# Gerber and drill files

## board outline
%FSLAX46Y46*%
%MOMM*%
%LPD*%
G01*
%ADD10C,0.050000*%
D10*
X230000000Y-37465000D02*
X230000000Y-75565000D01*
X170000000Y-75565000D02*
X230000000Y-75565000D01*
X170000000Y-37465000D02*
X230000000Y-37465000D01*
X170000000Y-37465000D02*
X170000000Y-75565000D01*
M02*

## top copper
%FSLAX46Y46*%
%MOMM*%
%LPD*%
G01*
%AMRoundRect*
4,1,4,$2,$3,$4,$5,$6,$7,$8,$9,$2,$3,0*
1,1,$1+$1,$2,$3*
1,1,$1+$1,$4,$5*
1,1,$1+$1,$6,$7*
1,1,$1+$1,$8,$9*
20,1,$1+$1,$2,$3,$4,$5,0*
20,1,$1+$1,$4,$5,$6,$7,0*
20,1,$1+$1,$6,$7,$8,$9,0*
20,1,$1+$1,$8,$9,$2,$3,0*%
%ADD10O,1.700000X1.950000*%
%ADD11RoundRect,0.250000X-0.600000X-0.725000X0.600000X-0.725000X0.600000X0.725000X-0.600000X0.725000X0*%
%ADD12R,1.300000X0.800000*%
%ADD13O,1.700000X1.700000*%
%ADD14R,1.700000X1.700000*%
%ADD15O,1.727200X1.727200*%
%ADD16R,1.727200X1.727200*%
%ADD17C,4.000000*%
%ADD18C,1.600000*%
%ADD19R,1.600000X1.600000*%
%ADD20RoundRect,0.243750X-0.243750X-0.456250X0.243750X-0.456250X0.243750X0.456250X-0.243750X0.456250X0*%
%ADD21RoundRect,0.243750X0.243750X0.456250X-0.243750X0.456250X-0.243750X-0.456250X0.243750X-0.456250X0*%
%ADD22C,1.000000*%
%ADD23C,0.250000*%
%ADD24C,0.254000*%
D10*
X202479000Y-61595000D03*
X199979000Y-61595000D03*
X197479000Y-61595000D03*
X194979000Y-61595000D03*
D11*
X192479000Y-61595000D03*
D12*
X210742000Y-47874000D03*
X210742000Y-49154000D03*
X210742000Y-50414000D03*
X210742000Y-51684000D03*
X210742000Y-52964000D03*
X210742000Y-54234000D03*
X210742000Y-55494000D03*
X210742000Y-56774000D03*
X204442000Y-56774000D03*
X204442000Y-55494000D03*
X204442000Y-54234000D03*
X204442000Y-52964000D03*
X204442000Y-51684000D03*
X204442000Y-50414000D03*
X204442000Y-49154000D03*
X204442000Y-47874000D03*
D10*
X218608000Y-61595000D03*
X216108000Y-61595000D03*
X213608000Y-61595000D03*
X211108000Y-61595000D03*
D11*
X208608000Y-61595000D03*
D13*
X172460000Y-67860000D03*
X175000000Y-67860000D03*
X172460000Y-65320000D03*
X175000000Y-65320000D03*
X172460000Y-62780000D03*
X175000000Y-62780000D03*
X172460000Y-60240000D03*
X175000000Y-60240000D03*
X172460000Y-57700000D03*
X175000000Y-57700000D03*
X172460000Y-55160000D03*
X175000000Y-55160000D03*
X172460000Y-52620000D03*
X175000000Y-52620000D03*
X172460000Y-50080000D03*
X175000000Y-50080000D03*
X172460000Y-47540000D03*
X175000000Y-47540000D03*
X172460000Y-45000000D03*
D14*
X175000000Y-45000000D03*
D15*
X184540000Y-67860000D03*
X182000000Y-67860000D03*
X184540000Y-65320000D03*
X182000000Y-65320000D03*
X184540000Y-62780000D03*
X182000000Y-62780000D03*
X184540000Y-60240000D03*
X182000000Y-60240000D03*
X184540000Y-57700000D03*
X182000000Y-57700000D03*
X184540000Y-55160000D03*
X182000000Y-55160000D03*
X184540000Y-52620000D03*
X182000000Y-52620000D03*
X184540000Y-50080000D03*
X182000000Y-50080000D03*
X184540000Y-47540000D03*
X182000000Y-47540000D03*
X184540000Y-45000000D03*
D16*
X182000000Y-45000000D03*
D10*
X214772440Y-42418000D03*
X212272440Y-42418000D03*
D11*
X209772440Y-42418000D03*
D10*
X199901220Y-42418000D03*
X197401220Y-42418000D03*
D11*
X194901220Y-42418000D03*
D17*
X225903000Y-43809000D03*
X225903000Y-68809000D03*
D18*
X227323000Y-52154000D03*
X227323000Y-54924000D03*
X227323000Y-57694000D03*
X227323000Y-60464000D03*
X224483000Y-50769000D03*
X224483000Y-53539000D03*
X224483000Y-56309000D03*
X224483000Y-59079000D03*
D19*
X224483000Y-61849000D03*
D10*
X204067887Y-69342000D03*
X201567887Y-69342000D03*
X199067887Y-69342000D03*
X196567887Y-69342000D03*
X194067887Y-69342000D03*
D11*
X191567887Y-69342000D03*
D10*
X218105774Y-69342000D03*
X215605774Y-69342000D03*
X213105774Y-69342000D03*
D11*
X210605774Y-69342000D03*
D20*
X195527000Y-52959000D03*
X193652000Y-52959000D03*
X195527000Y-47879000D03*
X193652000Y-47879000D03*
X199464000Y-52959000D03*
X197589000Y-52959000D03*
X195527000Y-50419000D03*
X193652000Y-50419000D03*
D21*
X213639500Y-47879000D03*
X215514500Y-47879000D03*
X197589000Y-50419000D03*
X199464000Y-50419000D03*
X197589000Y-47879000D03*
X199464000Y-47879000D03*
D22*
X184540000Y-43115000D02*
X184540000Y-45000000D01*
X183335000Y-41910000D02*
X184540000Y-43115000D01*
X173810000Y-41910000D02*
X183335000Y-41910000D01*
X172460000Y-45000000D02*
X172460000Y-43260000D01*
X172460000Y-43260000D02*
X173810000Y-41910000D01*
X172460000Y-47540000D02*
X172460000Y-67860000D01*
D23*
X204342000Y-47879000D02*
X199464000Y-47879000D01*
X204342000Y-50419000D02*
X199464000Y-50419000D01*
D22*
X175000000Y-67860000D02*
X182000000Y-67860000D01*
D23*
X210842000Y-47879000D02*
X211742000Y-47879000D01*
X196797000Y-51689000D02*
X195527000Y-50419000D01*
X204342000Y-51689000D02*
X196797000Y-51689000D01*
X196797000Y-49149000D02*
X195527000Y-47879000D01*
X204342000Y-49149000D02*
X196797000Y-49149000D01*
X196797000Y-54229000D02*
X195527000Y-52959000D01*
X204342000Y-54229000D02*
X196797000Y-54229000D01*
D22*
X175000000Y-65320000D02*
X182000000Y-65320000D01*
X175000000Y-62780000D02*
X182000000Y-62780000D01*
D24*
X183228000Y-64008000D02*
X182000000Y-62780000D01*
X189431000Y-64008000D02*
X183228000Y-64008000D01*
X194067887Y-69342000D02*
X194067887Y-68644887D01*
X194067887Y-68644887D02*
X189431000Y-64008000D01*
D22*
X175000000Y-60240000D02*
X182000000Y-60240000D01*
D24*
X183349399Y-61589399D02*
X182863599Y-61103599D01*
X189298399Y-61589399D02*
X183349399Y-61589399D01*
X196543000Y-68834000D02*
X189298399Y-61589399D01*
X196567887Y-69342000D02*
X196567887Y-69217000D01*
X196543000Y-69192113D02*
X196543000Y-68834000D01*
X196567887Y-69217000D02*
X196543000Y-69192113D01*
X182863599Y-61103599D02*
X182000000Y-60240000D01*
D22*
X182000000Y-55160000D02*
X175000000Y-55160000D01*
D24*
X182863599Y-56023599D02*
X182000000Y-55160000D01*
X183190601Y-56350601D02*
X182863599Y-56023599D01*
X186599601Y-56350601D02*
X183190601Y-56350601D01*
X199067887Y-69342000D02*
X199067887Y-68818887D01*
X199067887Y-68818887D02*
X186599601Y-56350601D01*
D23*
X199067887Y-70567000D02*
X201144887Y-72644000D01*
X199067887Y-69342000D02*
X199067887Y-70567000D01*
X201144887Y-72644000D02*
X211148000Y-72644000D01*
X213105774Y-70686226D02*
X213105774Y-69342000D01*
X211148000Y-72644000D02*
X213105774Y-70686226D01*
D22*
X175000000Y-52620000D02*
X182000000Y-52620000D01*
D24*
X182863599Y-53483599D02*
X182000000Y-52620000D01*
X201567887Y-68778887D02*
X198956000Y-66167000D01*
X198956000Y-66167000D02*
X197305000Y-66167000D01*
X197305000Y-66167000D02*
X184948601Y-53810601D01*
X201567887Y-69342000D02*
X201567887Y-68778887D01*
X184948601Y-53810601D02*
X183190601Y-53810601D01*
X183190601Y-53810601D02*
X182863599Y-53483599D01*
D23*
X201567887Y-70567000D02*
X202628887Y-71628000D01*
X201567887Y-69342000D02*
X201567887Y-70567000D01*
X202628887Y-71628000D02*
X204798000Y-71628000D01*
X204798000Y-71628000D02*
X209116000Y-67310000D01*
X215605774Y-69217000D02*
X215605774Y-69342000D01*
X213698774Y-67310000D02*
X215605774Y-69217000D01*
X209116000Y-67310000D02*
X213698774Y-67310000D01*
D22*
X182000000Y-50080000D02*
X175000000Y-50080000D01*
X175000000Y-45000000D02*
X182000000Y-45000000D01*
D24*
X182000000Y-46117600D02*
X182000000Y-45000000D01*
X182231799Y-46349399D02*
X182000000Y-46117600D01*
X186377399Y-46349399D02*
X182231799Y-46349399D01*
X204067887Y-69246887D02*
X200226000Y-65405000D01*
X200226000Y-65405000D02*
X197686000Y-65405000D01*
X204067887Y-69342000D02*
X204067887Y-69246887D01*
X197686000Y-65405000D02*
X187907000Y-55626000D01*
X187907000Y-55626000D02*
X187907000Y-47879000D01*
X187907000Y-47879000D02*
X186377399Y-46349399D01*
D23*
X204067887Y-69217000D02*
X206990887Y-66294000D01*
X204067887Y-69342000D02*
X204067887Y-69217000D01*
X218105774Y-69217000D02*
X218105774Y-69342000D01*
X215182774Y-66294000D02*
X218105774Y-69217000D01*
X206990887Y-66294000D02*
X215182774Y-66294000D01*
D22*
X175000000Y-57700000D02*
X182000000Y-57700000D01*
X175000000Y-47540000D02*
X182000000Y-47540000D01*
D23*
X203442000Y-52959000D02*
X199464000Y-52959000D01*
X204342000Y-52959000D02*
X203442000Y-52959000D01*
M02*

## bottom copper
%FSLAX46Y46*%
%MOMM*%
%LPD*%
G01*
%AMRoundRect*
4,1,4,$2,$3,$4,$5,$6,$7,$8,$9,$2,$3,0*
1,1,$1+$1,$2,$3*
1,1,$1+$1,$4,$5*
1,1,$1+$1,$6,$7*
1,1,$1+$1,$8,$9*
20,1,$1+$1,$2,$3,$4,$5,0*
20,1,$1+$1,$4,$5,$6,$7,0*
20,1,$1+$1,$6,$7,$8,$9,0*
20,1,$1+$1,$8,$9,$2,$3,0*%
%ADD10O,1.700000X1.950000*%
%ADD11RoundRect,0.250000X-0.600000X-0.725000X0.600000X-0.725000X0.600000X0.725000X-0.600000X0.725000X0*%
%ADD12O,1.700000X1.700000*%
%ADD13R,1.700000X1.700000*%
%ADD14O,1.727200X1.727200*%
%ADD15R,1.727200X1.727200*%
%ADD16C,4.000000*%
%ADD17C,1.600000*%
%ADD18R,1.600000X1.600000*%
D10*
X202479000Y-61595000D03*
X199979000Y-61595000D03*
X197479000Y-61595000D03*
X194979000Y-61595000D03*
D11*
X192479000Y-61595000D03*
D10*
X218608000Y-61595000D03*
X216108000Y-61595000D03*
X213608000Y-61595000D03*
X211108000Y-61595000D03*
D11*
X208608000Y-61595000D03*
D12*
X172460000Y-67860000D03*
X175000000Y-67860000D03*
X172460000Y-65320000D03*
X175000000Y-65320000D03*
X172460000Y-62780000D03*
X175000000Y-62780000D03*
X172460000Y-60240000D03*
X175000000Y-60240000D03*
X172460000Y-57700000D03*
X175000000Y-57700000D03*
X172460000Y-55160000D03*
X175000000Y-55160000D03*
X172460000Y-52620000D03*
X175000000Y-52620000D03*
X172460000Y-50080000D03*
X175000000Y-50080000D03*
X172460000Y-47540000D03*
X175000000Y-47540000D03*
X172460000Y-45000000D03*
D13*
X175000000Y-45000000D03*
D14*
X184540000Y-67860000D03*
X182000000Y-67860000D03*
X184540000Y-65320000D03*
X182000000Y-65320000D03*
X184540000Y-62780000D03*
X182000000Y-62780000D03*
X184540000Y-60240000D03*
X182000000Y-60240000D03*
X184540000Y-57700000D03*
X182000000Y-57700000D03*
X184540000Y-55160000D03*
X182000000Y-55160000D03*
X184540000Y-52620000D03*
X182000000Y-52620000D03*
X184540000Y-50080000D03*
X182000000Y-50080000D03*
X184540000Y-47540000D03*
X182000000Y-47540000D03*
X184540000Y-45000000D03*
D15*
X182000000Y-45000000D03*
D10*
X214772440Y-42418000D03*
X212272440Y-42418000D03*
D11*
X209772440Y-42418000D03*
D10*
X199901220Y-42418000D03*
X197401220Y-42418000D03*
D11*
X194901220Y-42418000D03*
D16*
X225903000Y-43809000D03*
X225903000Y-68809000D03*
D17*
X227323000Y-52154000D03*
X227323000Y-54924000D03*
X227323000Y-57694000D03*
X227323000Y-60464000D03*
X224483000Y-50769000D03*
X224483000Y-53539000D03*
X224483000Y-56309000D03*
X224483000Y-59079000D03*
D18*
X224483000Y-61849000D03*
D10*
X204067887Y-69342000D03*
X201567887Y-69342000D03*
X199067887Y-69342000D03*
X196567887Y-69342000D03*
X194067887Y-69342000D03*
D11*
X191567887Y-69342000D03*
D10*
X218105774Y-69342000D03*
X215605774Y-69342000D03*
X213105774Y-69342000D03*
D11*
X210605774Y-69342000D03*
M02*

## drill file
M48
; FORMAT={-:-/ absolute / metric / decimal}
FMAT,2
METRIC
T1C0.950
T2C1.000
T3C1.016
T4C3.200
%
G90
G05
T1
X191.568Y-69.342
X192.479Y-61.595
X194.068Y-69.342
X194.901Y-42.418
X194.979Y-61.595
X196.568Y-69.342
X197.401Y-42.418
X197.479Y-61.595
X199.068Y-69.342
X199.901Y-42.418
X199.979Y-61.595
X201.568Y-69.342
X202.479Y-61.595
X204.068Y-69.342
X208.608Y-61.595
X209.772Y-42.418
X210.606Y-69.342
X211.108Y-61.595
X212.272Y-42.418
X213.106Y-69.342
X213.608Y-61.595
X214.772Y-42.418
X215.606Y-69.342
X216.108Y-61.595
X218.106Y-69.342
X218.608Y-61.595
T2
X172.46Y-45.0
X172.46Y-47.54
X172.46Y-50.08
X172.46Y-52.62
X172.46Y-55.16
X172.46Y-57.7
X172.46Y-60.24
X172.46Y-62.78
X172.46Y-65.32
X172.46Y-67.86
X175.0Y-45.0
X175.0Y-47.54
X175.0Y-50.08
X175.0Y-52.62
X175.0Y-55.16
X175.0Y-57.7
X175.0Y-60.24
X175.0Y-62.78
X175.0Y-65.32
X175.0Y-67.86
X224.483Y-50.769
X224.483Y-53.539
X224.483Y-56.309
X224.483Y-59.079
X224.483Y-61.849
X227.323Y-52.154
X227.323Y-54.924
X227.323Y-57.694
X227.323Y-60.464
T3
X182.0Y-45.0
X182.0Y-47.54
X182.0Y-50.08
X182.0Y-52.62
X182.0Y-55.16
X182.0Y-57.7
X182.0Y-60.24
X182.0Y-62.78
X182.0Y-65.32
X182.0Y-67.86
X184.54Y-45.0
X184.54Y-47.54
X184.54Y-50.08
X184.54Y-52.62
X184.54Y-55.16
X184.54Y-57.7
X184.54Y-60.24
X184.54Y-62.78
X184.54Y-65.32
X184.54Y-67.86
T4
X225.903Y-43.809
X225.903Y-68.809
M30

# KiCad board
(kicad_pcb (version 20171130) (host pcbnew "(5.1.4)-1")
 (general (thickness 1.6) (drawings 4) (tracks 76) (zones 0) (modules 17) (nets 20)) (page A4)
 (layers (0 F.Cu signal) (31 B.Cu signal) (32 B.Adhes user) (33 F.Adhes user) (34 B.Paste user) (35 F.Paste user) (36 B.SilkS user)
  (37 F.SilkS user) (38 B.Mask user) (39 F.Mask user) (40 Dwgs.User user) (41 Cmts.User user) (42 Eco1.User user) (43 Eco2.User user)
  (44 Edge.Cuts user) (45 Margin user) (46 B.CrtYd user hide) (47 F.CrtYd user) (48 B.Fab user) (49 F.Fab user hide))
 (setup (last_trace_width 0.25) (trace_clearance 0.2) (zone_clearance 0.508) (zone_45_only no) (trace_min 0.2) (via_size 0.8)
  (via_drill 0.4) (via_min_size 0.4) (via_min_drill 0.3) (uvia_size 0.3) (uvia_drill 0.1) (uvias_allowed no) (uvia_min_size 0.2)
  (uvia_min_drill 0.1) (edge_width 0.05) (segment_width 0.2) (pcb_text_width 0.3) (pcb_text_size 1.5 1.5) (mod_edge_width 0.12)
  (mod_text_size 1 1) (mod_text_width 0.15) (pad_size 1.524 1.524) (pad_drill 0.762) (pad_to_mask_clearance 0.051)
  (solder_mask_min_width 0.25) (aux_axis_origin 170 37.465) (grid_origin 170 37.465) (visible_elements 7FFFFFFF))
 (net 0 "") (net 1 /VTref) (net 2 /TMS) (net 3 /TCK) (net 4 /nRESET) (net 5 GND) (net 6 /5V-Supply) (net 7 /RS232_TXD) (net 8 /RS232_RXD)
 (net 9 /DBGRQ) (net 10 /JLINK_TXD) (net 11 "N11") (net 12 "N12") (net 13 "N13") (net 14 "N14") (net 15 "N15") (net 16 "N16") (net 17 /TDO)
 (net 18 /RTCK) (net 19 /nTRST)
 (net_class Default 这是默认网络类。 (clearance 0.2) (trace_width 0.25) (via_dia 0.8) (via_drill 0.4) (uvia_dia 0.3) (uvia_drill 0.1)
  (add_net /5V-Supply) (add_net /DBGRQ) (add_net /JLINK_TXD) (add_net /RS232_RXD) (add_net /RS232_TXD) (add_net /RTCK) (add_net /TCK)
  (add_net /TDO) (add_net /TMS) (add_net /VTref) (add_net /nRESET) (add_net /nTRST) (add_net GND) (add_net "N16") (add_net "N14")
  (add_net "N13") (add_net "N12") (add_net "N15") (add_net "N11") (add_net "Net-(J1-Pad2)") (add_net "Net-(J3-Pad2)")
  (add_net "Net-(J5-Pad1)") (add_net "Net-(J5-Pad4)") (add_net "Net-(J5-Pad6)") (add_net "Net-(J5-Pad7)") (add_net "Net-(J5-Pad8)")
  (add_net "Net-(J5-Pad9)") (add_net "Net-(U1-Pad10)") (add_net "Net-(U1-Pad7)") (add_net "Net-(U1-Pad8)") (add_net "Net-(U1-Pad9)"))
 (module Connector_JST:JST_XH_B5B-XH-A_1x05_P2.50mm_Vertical (layer F.Cu) (at 192.479 61.595)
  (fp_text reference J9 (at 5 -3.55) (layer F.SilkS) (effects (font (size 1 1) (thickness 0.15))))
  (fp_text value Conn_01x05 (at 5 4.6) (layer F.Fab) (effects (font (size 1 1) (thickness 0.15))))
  (pad 5 thru_hole oval (at 10 0) (size 1.7 1.95) (drill 0.95) (layers *.Cu *.Mask) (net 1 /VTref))
  (pad 4 thru_hole oval (at 7.5 0) (size 1.7 1.95) (drill 0.95) (layers *.Cu *.Mask) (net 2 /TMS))
  (pad 3 thru_hole oval (at 5 0) (size 1.7 1.95) (drill 0.95) (layers *.Cu *.Mask) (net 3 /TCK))
  (pad 2 thru_hole oval (at 2.5 0) (size 1.7 1.95) (drill 0.95) (layers *.Cu *.Mask) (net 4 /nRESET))
  (pad 1 thru_hole roundrect (at 0 0) (size 1.7 1.95) (drill 0.95) (layers *.Cu *.Mask) (roundrect_rratio 0.147059) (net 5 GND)))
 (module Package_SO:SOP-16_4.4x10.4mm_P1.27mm (layer F.Cu) (at 207.592 52.324)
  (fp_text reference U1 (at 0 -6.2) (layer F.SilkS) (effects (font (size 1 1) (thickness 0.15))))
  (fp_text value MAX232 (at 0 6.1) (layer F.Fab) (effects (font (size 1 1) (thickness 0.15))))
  (pad 16 smd rect (at 3.15 -4.45) (size 1.3 0.8) (layers F.Cu F.Paste F.Mask) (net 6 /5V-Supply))
  (pad 15 smd rect (at 3.15 -3.17) (size 1.3 0.8) (layers F.Cu F.Paste F.Mask) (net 5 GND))
  (pad 14 smd rect (at 3.15 -1.91) (size 1.3 0.8) (layers F.Cu F.Paste F.Mask) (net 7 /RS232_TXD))
  (pad 13 smd rect (at 3.15 -0.64) (size 1.3 0.8) (layers F.Cu F.Paste F.Mask) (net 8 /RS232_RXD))
  (pad 12 smd rect (at 3.15 0.64) (size 1.3 0.8) (layers F.Cu F.Paste F.Mask) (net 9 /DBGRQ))
  (pad 11 smd rect (at 3.15 1.91) (size 1.3 0.8) (layers F.Cu F.Paste F.Mask) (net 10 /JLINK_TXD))
  (pad 10 smd rect (at 3.15 3.17) (size 1.3 0.8) (layers F.Cu F.Paste F.Mask))
  (pad 9 smd rect (at 3.15 4.45) (size 1.3 0.8) (layers F.Cu F.Paste F.Mask))
  (pad 8 smd rect (at -3.15 4.45) (size 1.3 0.8) (layers F.Cu F.Paste F.Mask))
  (pad 7 smd rect (at -3.15 3.17) (size 1.3 0.8) (layers F.Cu F.Paste F.Mask))
  (pad 6 smd rect (at -3.15 1.91) (size 1.3 0.8) (layers F.Cu F.Paste F.Mask) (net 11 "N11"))
  (pad 5 smd rect (at -3.15 0.64) (size 1.3 0.8) (layers F.Cu F.Paste F.Mask) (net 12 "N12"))
  (pad 4 smd rect (at -3.15 -0.64) (size 1.3 0.8) (layers F.Cu F.Paste F.Mask) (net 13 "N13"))
  (pad 3 smd rect (at -3.15 -1.91) (size 1.3 0.8) (layers F.Cu F.Paste F.Mask) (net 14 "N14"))
  (pad 2 smd rect (at -3.15 -3.17) (size 1.3 0.8) (layers F.Cu F.Paste F.Mask) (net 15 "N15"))
  (pad 1 smd rect (at -3.15 -4.45) (size 1.3 0.8) (layers F.Cu F.Paste F.Mask) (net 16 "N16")))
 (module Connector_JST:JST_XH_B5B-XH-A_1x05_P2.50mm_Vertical (layer F.Cu) (at 208.608 61.595)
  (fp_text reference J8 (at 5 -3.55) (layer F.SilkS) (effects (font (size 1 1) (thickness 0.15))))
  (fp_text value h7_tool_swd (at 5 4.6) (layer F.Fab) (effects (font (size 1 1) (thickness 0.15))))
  (pad 5 thru_hole oval (at 10 0) (size 1.7 1.95) (drill 0.95) (layers *.Cu *.Mask) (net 4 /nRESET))
  (pad 4 thru_hole oval (at 7.5 0) (size 1.7 1.95) (drill 0.95) (layers *.Cu *.Mask) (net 3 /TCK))
  (pad 3 thru_hole oval (at 5 0) (size 1.7 1.95) (drill 0.95) (layers *.Cu *.Mask) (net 2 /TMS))
  (pad 2 thru_hole oval (at 2.5 0) (size 1.7 1.95) (drill 0.95) (layers *.Cu *.Mask) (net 5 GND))
  (pad 1 thru_hole roundrect (at 0 0) (size 1.7 1.95) (drill 0.95) (layers *.Cu *.Mask) (roundrect_rratio 0.147059) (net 1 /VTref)))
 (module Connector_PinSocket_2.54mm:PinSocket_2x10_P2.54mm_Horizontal (layer F.Cu) (at 175 45)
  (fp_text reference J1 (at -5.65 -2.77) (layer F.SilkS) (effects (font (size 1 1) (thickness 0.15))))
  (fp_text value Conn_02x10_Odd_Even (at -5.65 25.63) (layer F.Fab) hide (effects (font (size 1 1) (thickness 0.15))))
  (pad 20 thru_hole oval (at -2.54 22.86) (size 1.7 1.7) (drill 1) (layers *.Cu *.Mask) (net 5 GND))
  (pad 19 thru_hole oval (at 0 22.86) (size 1.7 1.7) (drill 1) (layers *.Cu *.Mask) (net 6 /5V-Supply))
  (pad 18 thru_hole oval (at -2.54 20.32) (size 1.7 1.7) (drill 1) (layers *.Cu *.Mask) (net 5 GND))
  (pad 17 thru_hole oval (at 0 20.32) (size 1.7 1.7) (drill 1) (layers *.Cu *.Mask) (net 9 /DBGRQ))
  (pad 16 thru_hole oval (at -2.54 17.78) (size 1.7 1.7) (drill 1) (layers *.Cu *.Mask) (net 5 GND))
  (pad 15 thru_hole oval (at 0 17.78) (size 1.7 1.7) (drill 1) (layers *.Cu *.Mask) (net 4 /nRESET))
  (pad 14 thru_hole oval (at -2.54 15.24) (size 1.7 1.7) (drill 1) (layers *.Cu *.Mask) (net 5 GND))
  (pad 13 thru_hole oval (at 0 15.24) (size 1.7 1.7) (drill 1) (layers *.Cu *.Mask) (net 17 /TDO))
  (pad 12 thru_hole oval (at -2.54 12.7) (size 1.7 1.7) (drill 1) (layers *.Cu *.Mask) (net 5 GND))
  (pad 11 thru_hole oval (at 0 12.7) (size 1.7 1.7) (drill 1) (layers *.Cu *.Mask) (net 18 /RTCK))
  (pad 10 thru_hole oval (at -2.54 10.16) (size 1.7 1.7) (drill 1) (layers *.Cu *.Mask) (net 5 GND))
  (pad 9 thru_hole oval (at 0 10.16) (size 1.7 1.7) (drill 1) (layers *.Cu *.Mask) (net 3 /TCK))
  (pad 8 thru_hole oval (at -2.54 7.62) (size 1.7 1.7) (drill 1) (layers *.Cu *.Mask) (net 5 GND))
  (pad 7 thru_hole oval (at 0 7.62) (size 1.7 1.7) (drill 1) (layers *.Cu *.Mask) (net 2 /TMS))
  (pad 6 thru_hole oval (at -2.54 5.08) (size 1.7 1.7) (drill 1) (layers *.Cu *.Mask) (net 5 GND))
  (pad 5 thru_hole oval (at 0 5.08) (size 1.7 1.7) (drill 1) (layers *.Cu *.Mask) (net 10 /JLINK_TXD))
  (pad 4 thru_hole oval (at -2.54 2.54) (size 1.7 1.7) (drill 1) (layers *.Cu *.Mask) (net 5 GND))
  (pad 3 thru_hole oval (at 0 2.54) (size 1.7 1.7) (drill 1) (layers *.Cu *.Mask) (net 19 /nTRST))
  (pad 2 thru_hole oval (at -2.54 0) (size 1.7 1.7) (drill 1) (layers *.Cu *.Mask))
  (pad 1 thru_hole rect (at 0 0) (size 1.7 1.7) (drill 1) (layers *.Cu *.Mask) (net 1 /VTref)))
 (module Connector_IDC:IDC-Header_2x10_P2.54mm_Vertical (layer F.Cu) (at 182 45)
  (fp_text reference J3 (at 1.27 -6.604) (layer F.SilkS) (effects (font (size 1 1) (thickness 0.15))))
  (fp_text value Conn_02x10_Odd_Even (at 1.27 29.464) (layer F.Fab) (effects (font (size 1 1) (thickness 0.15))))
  (pad 20 thru_hole oval (at 2.54 22.86) (size 1.7272 1.7272) (drill 1.016) (layers *.Cu *.Mask) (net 5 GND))
  (pad 19 thru_hole oval (at 0 22.86) (size 1.7272 1.7272) (drill 1.016) (layers *.Cu *.Mask) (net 6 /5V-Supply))
  (pad 18 thru_hole oval (at 2.54 20.32) (size 1.7272 1.7272) (drill 1.016) (layers *.Cu *.Mask) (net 5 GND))
  (pad 17 thru_hole oval (at 0 20.32) (size 1.7272 1.7272) (drill 1.016) (layers *.Cu *.Mask) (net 9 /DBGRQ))
  (pad 16 thru_hole oval (at 2.54 17.78) (size 1.7272 1.7272) (drill 1.016) (layers *.Cu *.Mask) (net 5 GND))
  (pad 15 thru_hole oval (at 0 17.78) (size 1.7272 1.7272) (drill 1.016) (layers *.Cu *.Mask) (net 4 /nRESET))
  (pad 14 thru_hole oval (at 2.54 15.24) (size 1.7272 1.7272) (drill 1.016) (layers *.Cu *.Mask) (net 5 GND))
  (pad 13 thru_hole oval (at 0 15.24) (size 1.7272 1.7272) (drill 1.016) (layers *.Cu *.Mask) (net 17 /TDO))
  (pad 12 thru_hole oval (at 2.54 12.7) (size 1.7272 1.7272) (drill 1.016) (layers *.Cu *.Mask) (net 5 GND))
  (pad 11 thru_hole oval (at 0 12.7) (size 1.7272 1.7272) (drill 1.016) (layers *.Cu *.Mask) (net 18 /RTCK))
  (pad 10 thru_hole oval (at 2.54 10.16) (size 1.7272 1.7272) (drill 1.016) (layers *.Cu *.Mask) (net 5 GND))
  (pad 9 thru_hole oval (at 0 10.16) (size 1.7272 1.7272) (drill 1.016) (layers *.Cu *.Mask) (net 3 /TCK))
  (pad 8 thru_hole oval (at 2.54 7.62) (size 1.7272 1.7272) (drill 1.016) (layers *.Cu *.Mask) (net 5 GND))
  (pad 7 thru_hole oval (at 0 7.62) (size 1.7272 1.7272) (drill 1.016) (layers *.Cu *.Mask) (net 2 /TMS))
  (pad 6 thru_hole oval (at 2.54 5.08) (size 1.7272 1.7272) (drill 1.016) (layers *.Cu *.Mask) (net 5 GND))
  (pad 5 thru_hole oval (at 0 5.08) (size 1.7272 1.7272) (drill 1.016) (layers *.Cu *.Mask) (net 10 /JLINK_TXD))
  (pad 4 thru_hole oval (at 2.54 2.54) (size 1.7272 1.7272) (drill 1.016) (layers *.Cu *.Mask) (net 5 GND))
  (pad 3 thru_hole oval (at 0 2.54) (size 1.7272 1.7272) (drill 1.016) (layers *.Cu *.Mask) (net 19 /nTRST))
  (pad 2 thru_hole oval (at 2.54 0) (size 1.7272 1.7272) (drill 1.016) (layers *.Cu *.Mask))
  (pad 1 thru_hole rect (at 0 0) (size 1.7272 1.7272) (drill 1.016) (layers *.Cu *.Mask) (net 1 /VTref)))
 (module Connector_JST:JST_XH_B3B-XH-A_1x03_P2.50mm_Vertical (layer F.Cu) (at 209.77244 42.418)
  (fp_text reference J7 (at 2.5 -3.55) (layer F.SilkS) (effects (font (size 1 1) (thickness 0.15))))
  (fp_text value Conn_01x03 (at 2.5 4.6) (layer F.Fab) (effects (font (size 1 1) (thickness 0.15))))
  (pad 3 thru_hole oval (at 5 0) (size 1.7 1.95) (drill 0.95) (layers *.Cu *.Mask) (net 5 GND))
  (pad 2 thru_hole oval (at 2.5 0) (size 1.7 1.95) (drill 0.95) (layers *.Cu *.Mask) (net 8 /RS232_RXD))
  (pad 1 thru_hole roundrect (at 0 0) (size 1.7 1.95) (drill 0.95) (layers *.Cu *.Mask) (roundrect_rratio 0.147059) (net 7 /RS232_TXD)))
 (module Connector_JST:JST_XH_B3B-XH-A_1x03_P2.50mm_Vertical (layer F.Cu) (at 194.90122 42.418)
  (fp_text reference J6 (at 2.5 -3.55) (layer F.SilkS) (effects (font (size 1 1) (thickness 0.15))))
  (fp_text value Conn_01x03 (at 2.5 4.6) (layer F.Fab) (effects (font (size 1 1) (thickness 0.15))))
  (pad 3 thru_hole oval (at 5 0) (size 1.7 1.95) (drill 0.95) (layers *.Cu *.Mask) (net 5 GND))
  (pad 2 thru_hole oval (at 2.5 0) (size 1.7 1.95) (drill 0.95) (layers *.Cu *.Mask) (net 9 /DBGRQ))
  (pad 1 thru_hole roundrect (at 0 0) (size 1.7 1.95) (drill 0.95) (layers *.Cu *.Mask) (roundrect_rratio 0.147059) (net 10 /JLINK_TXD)))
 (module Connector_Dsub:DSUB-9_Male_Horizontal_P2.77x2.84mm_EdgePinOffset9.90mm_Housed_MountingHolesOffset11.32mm (layer F.Cu)
  (at 224.483 61.849 90)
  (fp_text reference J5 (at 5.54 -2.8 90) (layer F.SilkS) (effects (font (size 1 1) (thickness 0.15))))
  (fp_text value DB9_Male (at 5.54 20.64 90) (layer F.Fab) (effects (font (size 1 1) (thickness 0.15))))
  (pad 0 thru_hole circle (at 18.04 1.42 90) (size 4 4) (drill 3.2) (layers *.Cu *.Mask))
  (pad 0 thru_hole circle (at -6.96 1.42 90) (size 4 4) (drill 3.2) (layers *.Cu *.Mask))
  (pad 9 thru_hole circle (at 9.695 2.84 90) (size 1.6 1.6) (drill 1) (layers *.Cu *.Mask))
  (pad 8 thru_hole circle (at 6.925 2.84 90) (size 1.6 1.6) (drill 1) (layers *.Cu *.Mask))
  (pad 7 thru_hole circle (at 4.155 2.84 90) (size 1.6 1.6) (drill 1) (layers *.Cu *.Mask))
  (pad 6 thru_hole circle (at 1.385 2.84 90) (size 1.6 1.6) (drill 1) (layers *.Cu *.Mask))
  (pad 5 thru_hole circle (at 11.08 0 90) (size 1.6 1.6) (drill 1) (layers *.Cu *.Mask) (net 5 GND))
  (pad 4 thru_hole circle (at 8.31 0 90) (size 1.6 1.6) (drill 1) (layers *.Cu *.Mask))
  (pad 3 thru_hole circle (at 5.54 0 90) (size 1.6 1.6) (drill 1) (layers *.Cu *.Mask) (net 7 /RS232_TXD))
  (pad 2 thru_hole circle (at 2.77 0 90) (size 1.6 1.6) (drill 1) (layers *.Cu *.Mask) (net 8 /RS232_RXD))
  (pad 1 thru_hole rect (at 0 0 90) (size 1.6 1.6) (drill 1) (layers *.Cu *.Mask)))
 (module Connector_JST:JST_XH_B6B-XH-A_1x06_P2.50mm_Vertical (layer F.Cu) (at 191.567887 69.342)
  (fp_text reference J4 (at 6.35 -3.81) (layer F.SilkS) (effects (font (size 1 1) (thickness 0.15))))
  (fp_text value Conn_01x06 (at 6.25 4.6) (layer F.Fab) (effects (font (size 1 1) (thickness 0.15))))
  (pad 6 thru_hole oval (at 12.5 0) (size 1.7 1.95) (drill 0.95) (layers *.Cu *.Mask) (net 1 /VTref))
  (pad 5 thru_hole oval (at 10 0) (size 1.7 1.95) (drill 0.95) (layers *.Cu *.Mask) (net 2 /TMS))
  (pad 4 thru_hole oval (at 7.5 0) (size 1.7 1.95) (drill 0.95) (layers *.Cu *.Mask) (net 3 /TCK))
  (pad 3 thru_hole oval (at 5 0) (size 1.7 1.95) (drill 0.95) (layers *.Cu *.Mask) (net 17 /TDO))
  (pad 2 thru_hole oval (at 2.5 0) (size 1.7 1.95) (drill 0.95) (layers *.Cu *.Mask) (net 4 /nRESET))
  (pad 1 thru_hole roundrect (at 0 0) (size 1.7 1.95) (drill 0.95) (layers *.Cu *.Mask) (roundrect_rratio 0.147059) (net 5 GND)))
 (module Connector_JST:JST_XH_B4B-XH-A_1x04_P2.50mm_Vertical (layer F.Cu) (at 210.605774 69.342)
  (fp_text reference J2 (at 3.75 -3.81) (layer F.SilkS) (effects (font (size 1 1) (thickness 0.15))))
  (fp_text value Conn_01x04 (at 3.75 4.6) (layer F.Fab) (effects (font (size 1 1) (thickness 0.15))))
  (pad 4 thru_hole oval (at 7.5 0) (size 1.7 1.95) (drill 0.95) (layers *.Cu *.Mask) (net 1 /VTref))
  (pad 3 thru_hole oval (at 5 0) (size 1.7 1.95) (drill 0.95) (layers *.Cu *.Mask) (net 2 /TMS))
  (pad 2 thru_hole oval (at 2.5 0) (size 1.7 1.95) (drill 0.95) (layers *.Cu *.Mask) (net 3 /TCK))
  (pad 1 thru_hole roundrect (at 0 0) (size 1.7 1.95) (drill 0.95) (layers *.Cu *.Mask) (roundrect_rratio 0.147059) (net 5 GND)))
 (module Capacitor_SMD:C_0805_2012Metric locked (layer F.Cu) (at 194.5895 52.959)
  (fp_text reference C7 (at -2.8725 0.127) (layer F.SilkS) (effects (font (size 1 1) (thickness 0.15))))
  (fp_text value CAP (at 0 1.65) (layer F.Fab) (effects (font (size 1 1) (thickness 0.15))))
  (pad 2 smd roundrect (at 0.9375 0) (size 0.975 1.4) (layers F.Cu F.Paste F.Mask) (roundrect_rratio 0.25) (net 11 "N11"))
  (pad 1 smd roundrect (at -0.9375 0) (size 0.975 1.4) (layers F.Cu F.Paste F.Mask) (roundrect_rratio 0.25) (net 5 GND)))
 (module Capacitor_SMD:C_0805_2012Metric (layer F.Cu) (at 194.5895 47.879)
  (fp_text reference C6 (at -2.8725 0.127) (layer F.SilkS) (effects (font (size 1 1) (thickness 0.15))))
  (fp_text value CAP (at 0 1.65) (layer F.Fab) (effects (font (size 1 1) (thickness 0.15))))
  (pad 2 smd roundrect (at 0.9375 0) (size 0.975 1.4) (layers F.Cu F.Paste F.Mask) (roundrect_rratio 0.25) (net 15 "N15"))
  (pad 1 smd roundrect (at -0.9375 0) (size 0.975 1.4) (layers F.Cu F.Paste F.Mask) (roundrect_rratio 0.25) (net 5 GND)))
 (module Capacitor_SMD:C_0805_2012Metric (layer F.Cu) (at 198.5265 52.959)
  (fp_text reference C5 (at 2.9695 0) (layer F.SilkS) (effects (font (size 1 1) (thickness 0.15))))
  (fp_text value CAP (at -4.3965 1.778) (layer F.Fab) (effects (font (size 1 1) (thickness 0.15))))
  (pad 2 smd roundrect (at 0.9375 0) (size 0.975 1.4) (layers F.Cu F.Paste F.Mask) (roundrect_rratio 0.25) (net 12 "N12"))
  (pad 1 smd roundrect (at -0.9375 0) (size 0.975 1.4) (layers F.Cu F.Paste F.Mask) (roundrect_rratio 0.25) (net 5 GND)))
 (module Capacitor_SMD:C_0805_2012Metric (layer F.Cu) (at 194.5895 50.419)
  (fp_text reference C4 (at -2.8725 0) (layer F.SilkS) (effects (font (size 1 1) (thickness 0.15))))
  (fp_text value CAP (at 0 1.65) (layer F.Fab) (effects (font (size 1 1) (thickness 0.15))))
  (pad 2 smd roundrect (at 0.9375 0) (size 0.975 1.4) (layers F.Cu F.Paste F.Mask) (roundrect_rratio 0.25) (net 13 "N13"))
  (pad 1 smd roundrect (at -0.9375 0) (size 0.975 1.4) (layers F.Cu F.Paste F.Mask) (roundrect_rratio 0.25) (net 5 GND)))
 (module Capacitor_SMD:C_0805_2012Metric (layer F.Cu) (at 214.577 47.879 180)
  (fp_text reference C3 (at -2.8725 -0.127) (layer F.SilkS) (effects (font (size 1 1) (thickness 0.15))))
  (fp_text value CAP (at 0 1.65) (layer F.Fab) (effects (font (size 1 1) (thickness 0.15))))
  (pad 2 smd roundrect (at 0.9375 0 180) (size 0.975 1.4) (layers F.Cu F.Paste F.Mask) (roundrect_rratio 0.25) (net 6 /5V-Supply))
  (pad 1 smd roundrect (at -0.9375 0 180) (size 0.975 1.4) (layers F.Cu F.Paste F.Mask) (roundrect_rratio 0.25) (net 5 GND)))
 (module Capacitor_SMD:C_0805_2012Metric (layer F.Cu) (at 198.5265 50.419 180)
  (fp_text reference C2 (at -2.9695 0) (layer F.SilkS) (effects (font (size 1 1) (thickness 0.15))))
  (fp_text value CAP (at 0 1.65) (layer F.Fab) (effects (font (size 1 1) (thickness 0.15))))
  (pad 2 smd roundrect (at 0.9375 0 180) (size 0.975 1.4) (layers F.Cu F.Paste F.Mask) (roundrect_rratio 0.25) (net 5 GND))
  (pad 1 smd roundrect (at -0.9375 0 180) (size 0.975 1.4) (layers F.Cu F.Paste F.Mask) (roundrect_rratio 0.25) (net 14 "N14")))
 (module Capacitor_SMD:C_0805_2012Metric (layer F.Cu) (at 198.5265 47.879 180)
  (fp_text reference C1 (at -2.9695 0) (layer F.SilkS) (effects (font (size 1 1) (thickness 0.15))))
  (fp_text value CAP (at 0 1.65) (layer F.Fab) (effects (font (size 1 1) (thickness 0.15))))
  (pad 2 smd roundrect (at 0.9375 0 180) (size 0.975 1.4) (layers F.Cu F.Paste F.Mask) (roundrect_rratio 0.25) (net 5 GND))
  (pad 1 smd roundrect (at -0.9375 0 180) (size 0.975 1.4) (layers F.Cu F.Paste F.Mask) (roundrect_rratio 0.25) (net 16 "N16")))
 (gr_line (start 230 37.465) (end 230 75.565) (layer Edge.Cuts) (width 0.05))
 (gr_line (start 170 75.565) (end 230 75.565) (layer Edge.Cuts) (width 0.05))
 (gr_line (start 170 37.465) (end 230 37.465) (layer Edge.Cuts) (width 0.05))
 (gr_line (start 170 37.465) (end 170 75.565) (layer Edge.Cuts) (width 0.05))
 (segment (start 184.54 43.115) (end 184.54 45) (width 1) (layer F.Cu) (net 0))
 (segment (start 183.335 41.91) (end 184.54 43.115) (width 1) (layer F.Cu) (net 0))
 (segment (start 173.81 41.91) (end 183.335 41.91) (width 1) (layer F.Cu) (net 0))
 (segment (start 172.46 45) (end 172.46 43.26) (width 1) (layer F.Cu) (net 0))
 (segment (start 172.46 43.26) (end 173.81 41.91) (width 1) (layer F.Cu) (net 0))
 (segment (start 172.46 47.54) (end 172.46 67.86) (width 1) (layer F.Cu) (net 5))
 (segment (start 204.342 47.879) (end 199.464 47.879) (width 0.25) (layer F.Cu) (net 16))
 (segment (start 204.342 50.419) (end 199.464 50.419) (width 0.25) (layer F.Cu) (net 14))
 (segment (start 175 67.86) (end 182 67.86) (width 1) (layer F.Cu) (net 6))
 (segment (start 210.842 47.879) (end 211.742 47.879) (width 0.25) (layer F.Cu) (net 6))
 (segment (start 196.797 51.689) (end 195.527 50.419) (width 0.25) (layer F.Cu) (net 13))
 (segment (start 204.342 51.689) (end 196.797 51.689) (width 0.25) (layer F.Cu) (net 13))
 (segment (start 196.797 49.149) (end 195.527 47.879) (width 0.25) (layer F.Cu) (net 15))
 (segment (start 204.342 49.149) (end 196.797 49.149) (width 0.25) (layer F.Cu) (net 15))
 (segment (start 196.797 54.229) (end 195.527 52.959) (width 0.25) (layer F.Cu) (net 11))
 (segment (start 204.342 54.229) (end 196.797 54.229) (width 0.25) (layer F.Cu) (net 11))
 (segment (start 175 65.32) (end 182 65.32) (width 1) (layer F.Cu) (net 9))
 (segment (start 175 62.78) (end 182 62.78) (width 1) (layer F.Cu) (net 4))
 (segment (start 183.228 64.008) (end 182 62.78) (width 0.254) (layer F.Cu) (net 4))
 (segment (start 189.431 64.008) (end 183.228 64.008) (width 0.254) (layer F.Cu) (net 4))
 (segment (start 194.067887 69.342) (end 194.067887 68.644887) (width 0.254) (layer F.Cu) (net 4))
 (segment (start 194.067887 68.644887) (end 189.431 64.008) (width 0.254) (layer F.Cu) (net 4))
 (segment (start 175 60.24) (end 182 60.24) (width 1) (layer F.Cu) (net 17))
 (segment (start 183.349399 61.589399) (end 182.863599 61.103599) (width 0.254) (layer F.Cu) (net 17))
 (segment (start 189.298399 61.589399) (end 183.349399 61.589399) (width 0.254) (layer F.Cu) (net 17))
 (segment (start 196.543 68.834) (end 189.298399 61.589399) (width 0.254) (layer F.Cu) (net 17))
 (segment (start 196.567887 69.342) (end 196.567887 69.217) (width 0.254) (layer F.Cu) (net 17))
 (segment (start 196.543 69.192113) (end 196.543 68.834) (width 0.254) (layer F.Cu) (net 17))
 (segment (start 196.567887 69.217) (end 196.543 69.192113) (width 0.254) (layer F.Cu) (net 17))
 (segment (start 182.863599 61.103599) (end 182 60.24) (width 0.254) (layer F.Cu) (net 17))
 (segment (start 182 55.16) (end 175 55.16) (width 1) (layer F.Cu) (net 3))
 (segment (start 182.863599 56.023599) (end 182 55.16) (width 0.254) (layer F.Cu) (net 3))
 (segment (start 183.190601 56.350601) (end 182.863599 56.023599) (width 0.254) (layer F.Cu) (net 3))
 (segment (start 186.599601 56.350601) (end 183.190601 56.350601) (width 0.254) (layer F.Cu) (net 3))
 (segment (start 199.067887 69.342) (end 199.067887 68.818887) (width 0.254) (layer F.Cu) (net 3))
 (segment (start 199.067887 68.818887) (end 186.599601 56.350601) (width 0.254) (layer F.Cu) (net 3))
 (segment (start 199.067887 70.567) (end 201.144887 72.644) (width 0.25) (layer F.Cu) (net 3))
 (segment (start 199.067887 69.342) (end 199.067887 70.567) (width 0.25) (layer F.Cu) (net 3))
 (segment (start 201.144887 72.644) (end 211.148 72.644) (width 0.25) (layer F.Cu) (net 3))
 (segment (start 213.105774 70.686226) (end 213.105774 69.342) (width 0.25) (layer F.Cu) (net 3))
 (segment (start 211.148 72.644) (end 213.105774 70.686226) (width 0.25) (layer F.Cu) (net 3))
 (segment (start 175 52.62) (end 182 52.62) (width 1) (layer F.Cu) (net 2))
 (segment (start 182.863599 53.483599) (end 182 52.62) (width 0.254) (layer F.Cu) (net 2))
 (segment (start 201.567887 68.778887) (end 198.956 66.167) (width 0.254) (layer F.Cu) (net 2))
 (segment (start 198.956 66.167) (end 197.305 66.167) (width 0.254) (layer F.Cu) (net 2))
 (segment (start 197.305 66.167) (end 184.948601 53.810601) (width 0.254) (layer F.Cu) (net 2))
 (segment (start 201.567887 69.342) (end 201.567887 68.778887) (width 0.254) (layer F.Cu) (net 2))
 (segment (start 184.948601 53.810601) (end 183.190601 53.810601) (width 0.254) (layer F.Cu) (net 2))
 (segment (start 183.190601 53.810601) (end 182.863599 53.483599) (width 0.254) (layer F.Cu) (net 2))
 (segment (start 201.567887 70.567) (end 202.628887 71.628) (width 0.25) (layer F.Cu) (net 2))
 (segment (start 201.567887 69.342) (end 201.567887 70.567) (width 0.25) (layer F.Cu) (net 2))
 (segment (start 202.628887 71.628) (end 204.798 71.628) (width 0.25) (layer F.Cu) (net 2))
 (segment (start 204.798 71.628) (end 209.116 67.31) (width 0.25) (layer F.Cu) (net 2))
 (segment (start 215.605774 69.217) (end 215.605774 69.342) (width 0.25) (layer F.Cu) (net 2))
 (segment (start 213.698774 67.31) (end 215.605774 69.217) (width 0.25) (layer F.Cu) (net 2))
 (segment (start 209.116 67.31) (end 213.698774 67.31) (width 0.25) (layer F.Cu) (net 2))
 (segment (start 182 50.08) (end 175 50.08) (width 1) (layer F.Cu) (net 10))
 (segment (start 175 45) (end 182 45) (width 1) (layer F.Cu) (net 1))
 (segment (start 182 46.1176) (end 182 45) (width 0.254) (layer F.Cu) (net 1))
 (segment (start 182.231799 46.349399) (end 182 46.1176) (width 0.254) (layer F.Cu) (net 1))
 (segment (start 186.377399 46.349399) (end 182.231799 46.349399) (width 0.254) (layer F.Cu) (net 1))
 (segment (start 204.067887 69.246887) (end 200.226 65.405) (width 0.254) (layer F.Cu) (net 1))
 (segment (start 200.226 65.405) (end 197.686 65.405) (width 0.254) (layer F.Cu) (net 1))
 (segment (start 204.067887 69.342) (end 204.067887 69.246887) (width 0.254) (layer F.Cu) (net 1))
 (segment (start 197.686 65.405) (end 187.907 55.626) (width 0.254) (layer F.Cu) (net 1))
 (segment (start 187.907 55.626) (end 187.907 47.879) (width 0.254) (layer F.Cu) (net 1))
 (segment (start 187.907 47.879) (end 186.377399 46.349399) (width 0.254) (layer F.Cu) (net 1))
 (segment (start 204.067887 69.217) (end 206.990887 66.294) (width 0.25) (layer F.Cu) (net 1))
 (segment (start 204.067887 69.342) (end 204.067887 69.217) (width 0.25) (layer F.Cu) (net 1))
 (segment (start 218.105774 69.217) (end 218.105774 69.342) (width 0.25) (layer F.Cu) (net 1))
 (segment (start 215.182774 66.294) (end 218.105774 69.217) (width 0.25) (layer F.Cu) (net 1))
 (segment (start 206.990887 66.294) (end 215.182774 66.294) (width 0.25) (layer F.Cu) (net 1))
 (segment (start 175 57.7) (end 182 57.7) (width 1) (layer F.Cu) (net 18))
 (segment (start 175 47.54) (end 182 47.54) (width 1) (layer F.Cu) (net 19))
 (segment (start 203.442 52.959) (end 199.464 52.959) (width 0.25) (layer F.Cu) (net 12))
 (segment (start 204.342 52.959) (end 203.442 52.959) (width 0.25) (layer F.Cu) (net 12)))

